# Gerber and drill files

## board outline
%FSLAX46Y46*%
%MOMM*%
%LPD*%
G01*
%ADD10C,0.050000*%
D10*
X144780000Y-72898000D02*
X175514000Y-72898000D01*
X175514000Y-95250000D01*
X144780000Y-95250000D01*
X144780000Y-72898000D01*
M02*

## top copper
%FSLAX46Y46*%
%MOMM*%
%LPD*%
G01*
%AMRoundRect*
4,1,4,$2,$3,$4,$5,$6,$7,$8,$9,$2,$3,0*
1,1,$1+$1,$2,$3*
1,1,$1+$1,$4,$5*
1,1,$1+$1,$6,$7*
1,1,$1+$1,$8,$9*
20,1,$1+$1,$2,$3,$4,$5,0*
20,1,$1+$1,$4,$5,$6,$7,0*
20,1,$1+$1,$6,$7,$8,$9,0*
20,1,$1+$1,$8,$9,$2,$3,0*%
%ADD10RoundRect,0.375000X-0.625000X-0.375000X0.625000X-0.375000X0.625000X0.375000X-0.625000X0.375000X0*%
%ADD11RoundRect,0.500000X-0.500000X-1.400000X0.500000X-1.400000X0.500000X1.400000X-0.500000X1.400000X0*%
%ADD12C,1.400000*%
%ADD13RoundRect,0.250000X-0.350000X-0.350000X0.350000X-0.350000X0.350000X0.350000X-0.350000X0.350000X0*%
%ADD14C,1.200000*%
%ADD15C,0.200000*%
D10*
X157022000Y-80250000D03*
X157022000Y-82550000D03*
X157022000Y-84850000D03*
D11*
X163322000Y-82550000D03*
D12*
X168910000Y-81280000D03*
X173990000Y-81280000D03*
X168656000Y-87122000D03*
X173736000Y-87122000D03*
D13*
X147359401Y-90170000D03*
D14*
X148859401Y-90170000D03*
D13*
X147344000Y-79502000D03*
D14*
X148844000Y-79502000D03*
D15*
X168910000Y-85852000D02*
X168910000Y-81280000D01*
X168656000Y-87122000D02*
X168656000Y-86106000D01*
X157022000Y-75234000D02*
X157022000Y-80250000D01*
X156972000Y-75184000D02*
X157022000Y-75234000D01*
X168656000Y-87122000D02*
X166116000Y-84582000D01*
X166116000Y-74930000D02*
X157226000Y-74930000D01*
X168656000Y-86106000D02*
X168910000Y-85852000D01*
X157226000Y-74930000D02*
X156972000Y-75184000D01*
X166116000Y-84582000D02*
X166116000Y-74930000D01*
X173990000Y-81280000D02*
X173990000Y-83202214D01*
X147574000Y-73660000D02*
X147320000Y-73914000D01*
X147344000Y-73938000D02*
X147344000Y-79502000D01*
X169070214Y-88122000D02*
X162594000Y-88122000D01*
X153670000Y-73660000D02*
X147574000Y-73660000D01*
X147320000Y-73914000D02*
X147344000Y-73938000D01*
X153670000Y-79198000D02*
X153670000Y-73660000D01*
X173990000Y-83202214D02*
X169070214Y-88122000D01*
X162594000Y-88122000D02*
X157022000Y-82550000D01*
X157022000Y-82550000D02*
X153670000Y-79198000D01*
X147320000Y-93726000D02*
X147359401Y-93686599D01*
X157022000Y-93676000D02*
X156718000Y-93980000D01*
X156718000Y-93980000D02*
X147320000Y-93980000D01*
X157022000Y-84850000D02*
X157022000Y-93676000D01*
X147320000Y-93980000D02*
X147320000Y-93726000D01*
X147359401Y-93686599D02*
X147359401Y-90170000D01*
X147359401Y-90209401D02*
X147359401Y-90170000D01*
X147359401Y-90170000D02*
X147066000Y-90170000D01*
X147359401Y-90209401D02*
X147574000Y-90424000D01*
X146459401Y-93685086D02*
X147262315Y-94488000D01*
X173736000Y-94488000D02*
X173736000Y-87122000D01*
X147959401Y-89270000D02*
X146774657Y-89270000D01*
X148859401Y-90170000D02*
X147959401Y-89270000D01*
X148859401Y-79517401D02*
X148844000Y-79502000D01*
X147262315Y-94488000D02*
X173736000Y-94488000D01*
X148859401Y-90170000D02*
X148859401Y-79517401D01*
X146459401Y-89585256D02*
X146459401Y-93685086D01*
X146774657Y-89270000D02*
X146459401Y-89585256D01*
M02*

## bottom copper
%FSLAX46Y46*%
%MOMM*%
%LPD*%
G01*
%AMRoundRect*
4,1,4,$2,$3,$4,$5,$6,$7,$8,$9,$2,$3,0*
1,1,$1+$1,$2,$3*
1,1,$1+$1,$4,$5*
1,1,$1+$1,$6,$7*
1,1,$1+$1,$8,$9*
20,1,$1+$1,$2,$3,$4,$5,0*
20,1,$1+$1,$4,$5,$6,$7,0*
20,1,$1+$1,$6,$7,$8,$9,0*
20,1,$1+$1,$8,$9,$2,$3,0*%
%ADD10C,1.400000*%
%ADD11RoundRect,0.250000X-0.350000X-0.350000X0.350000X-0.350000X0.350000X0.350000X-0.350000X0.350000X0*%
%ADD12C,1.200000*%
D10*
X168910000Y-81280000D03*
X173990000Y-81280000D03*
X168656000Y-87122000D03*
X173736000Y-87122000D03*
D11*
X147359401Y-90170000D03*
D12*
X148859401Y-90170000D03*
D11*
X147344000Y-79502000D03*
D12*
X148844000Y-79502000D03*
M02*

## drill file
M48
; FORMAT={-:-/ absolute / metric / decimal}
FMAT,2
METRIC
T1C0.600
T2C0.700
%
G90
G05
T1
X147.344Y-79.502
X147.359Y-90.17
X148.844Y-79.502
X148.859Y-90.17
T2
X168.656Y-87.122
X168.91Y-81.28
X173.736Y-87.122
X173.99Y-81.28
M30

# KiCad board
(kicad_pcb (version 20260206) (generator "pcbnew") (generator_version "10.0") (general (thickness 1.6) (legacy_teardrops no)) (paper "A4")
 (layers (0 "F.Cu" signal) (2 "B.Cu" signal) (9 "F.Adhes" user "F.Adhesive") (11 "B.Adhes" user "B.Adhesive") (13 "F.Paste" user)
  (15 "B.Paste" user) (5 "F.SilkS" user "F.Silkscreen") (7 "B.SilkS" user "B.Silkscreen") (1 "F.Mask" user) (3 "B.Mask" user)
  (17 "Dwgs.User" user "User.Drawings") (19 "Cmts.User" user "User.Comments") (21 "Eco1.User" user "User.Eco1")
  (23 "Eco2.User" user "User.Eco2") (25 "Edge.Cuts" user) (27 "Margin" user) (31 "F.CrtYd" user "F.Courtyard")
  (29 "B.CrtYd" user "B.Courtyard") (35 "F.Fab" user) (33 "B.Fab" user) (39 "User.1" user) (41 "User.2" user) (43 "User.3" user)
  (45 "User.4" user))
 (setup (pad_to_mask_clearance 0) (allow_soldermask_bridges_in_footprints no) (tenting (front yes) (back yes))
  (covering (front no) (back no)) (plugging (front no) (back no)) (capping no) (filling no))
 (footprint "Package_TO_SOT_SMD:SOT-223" (layer "F.Cu") (at 160.172 82.55)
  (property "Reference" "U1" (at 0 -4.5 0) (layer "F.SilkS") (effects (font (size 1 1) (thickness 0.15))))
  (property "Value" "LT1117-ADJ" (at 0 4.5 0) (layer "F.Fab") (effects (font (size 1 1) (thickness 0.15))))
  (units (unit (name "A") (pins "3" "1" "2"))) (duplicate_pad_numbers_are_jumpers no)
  (pad "1" smd roundrect (at -3.15 -2.3) (size 2 1.5) (layers "F.Cu" "F.Mask" "F.Paste") (roundrect_rratio 0.25) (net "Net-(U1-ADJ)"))
  (pad "2" smd roundrect (at -3.15 0) (size 2 1.5) (layers "F.Cu" "F.Mask" "F.Paste") (roundrect_rratio 0.25) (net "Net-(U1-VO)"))
  (pad "3" smd roundrect (at -3.15 2.3) (size 2 1.5) (layers "F.Cu" "F.Mask" "F.Paste") (roundrect_rratio 0.25) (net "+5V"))
  (pad "4" smd roundrect (at 3.15 0) (size 2 3.8) (layers "F.Cu" "F.Mask" "F.Paste") (roundrect_rratio 0.25)))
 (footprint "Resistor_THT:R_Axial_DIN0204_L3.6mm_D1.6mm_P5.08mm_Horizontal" (layer "F.Cu") (at 168.91 81.28)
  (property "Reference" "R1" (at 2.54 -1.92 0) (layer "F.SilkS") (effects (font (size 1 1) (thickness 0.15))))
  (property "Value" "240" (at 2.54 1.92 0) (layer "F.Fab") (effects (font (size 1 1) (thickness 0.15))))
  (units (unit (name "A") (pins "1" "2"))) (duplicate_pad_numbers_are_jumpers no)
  (pad "1" thru_hole circle (at 0 0) (size 1.4 1.4) (drill 0.7) (layers "*.Cu" "*.Mask") (remove_unused_layers no) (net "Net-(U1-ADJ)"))
  (pad "2" thru_hole circle (at 5.08 0) (size 1.4 1.4) (drill 0.7) (layers "*.Cu" "*.Mask") (remove_unused_layers no) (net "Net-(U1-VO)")))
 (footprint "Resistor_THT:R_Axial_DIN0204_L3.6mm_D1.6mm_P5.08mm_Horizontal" (layer "F.Cu") (at 168.656 87.122)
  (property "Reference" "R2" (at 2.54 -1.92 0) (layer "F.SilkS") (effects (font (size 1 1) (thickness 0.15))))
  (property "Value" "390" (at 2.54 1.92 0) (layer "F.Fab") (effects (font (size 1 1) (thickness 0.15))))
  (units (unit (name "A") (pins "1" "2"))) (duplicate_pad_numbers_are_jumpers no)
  (pad "1" thru_hole circle (at 0 0) (size 1.4 1.4) (drill 0.7) (layers "*.Cu" "*.Mask") (remove_unused_layers no) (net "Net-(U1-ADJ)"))
  (pad "2" thru_hole circle (at 5.08 0) (size 1.4 1.4) (drill 0.7) (layers "*.Cu" "*.Mask") (remove_unused_layers no) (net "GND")))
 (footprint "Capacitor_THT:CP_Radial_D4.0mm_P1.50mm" (layer "F.Cu") (at 147.359401 90.17)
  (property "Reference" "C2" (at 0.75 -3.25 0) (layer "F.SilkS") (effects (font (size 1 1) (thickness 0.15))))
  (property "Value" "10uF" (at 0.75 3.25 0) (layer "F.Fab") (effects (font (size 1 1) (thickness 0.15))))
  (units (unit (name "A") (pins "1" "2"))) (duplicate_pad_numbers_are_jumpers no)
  (pad "1" thru_hole roundrect (at 0 0) (size 1.2 1.2) (drill 0.6) (layers "*.Cu" "*.Mask") (remove_unused_layers no)
   (roundrect_rratio 0.208333) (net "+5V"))
  (pad "2" thru_hole circle (at 1.5 0) (size 1.2 1.2) (drill 0.6) (layers "*.Cu" "*.Mask") (remove_unused_layers no) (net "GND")))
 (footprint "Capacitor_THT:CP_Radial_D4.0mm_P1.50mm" (layer "F.Cu") (at 147.344 79.502)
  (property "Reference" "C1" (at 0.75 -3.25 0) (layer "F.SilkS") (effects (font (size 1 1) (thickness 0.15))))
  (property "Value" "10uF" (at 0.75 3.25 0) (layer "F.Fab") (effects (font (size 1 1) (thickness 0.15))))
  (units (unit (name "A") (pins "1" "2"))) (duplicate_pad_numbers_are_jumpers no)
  (pad "1" thru_hole roundrect (at 0 0) (size 1.2 1.2) (drill 0.6) (layers "*.Cu" "*.Mask") (remove_unused_layers no)
   (roundrect_rratio 0.208333) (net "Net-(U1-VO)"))
  (pad "2" thru_hole circle (at 1.5 0) (size 1.2 1.2) (drill 0.6) (layers "*.Cu" "*.Mask") (remove_unused_layers no) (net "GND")))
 (gr_rect (start 144.78 72.898) (end 175.514 95.25) (stroke (width 0.05) (type default)) (fill no) (layer "Edge.Cuts"))
 (segment (start 168.91 85.852) (end 168.91 81.28) (width 0.2) (layer "F.Cu") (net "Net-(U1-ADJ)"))
 (segment (start 168.656 87.122) (end 168.656 86.106) (width 0.2) (layer "F.Cu") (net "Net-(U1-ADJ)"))
 (segment (start 157.022 75.234) (end 157.022 80.25) (width 0.2) (layer "F.Cu") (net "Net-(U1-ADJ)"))
 (segment (start 156.972 75.184) (end 157.022 75.234) (width 0.2) (layer "F.Cu") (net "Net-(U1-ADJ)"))
 (segment (start 168.656 87.122) (end 166.116 84.582) (width 0.2) (layer "F.Cu") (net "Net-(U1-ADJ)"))
 (segment (start 166.116 74.93) (end 157.226 74.93) (width 0.2) (layer "F.Cu") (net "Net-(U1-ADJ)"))
 (segment (start 168.656 86.106) (end 168.91 85.852) (width 0.2) (layer "F.Cu") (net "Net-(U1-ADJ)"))
 (segment (start 157.226 74.93) (end 156.972 75.184) (width 0.2) (layer "F.Cu") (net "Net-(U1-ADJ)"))
 (segment (start 166.116 84.582) (end 166.116 74.93) (width 0.2) (layer "F.Cu") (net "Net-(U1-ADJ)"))
 (segment (start 173.99 81.28) (end 173.99 83.202214) (width 0.2) (layer "F.Cu") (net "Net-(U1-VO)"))
 (segment (start 147.574 73.66) (end 147.32 73.914) (width 0.2) (layer "F.Cu") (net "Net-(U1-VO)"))
 (segment (start 147.344 73.938) (end 147.344 79.502) (width 0.2) (layer "F.Cu") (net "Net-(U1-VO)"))
 (segment (start 169.070214 88.122) (end 162.594 88.122) (width 0.2) (layer "F.Cu") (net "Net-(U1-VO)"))
 (segment (start 153.67 73.66) (end 147.574 73.66) (width 0.2) (layer "F.Cu") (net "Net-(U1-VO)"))
 (segment (start 147.32 73.914) (end 147.344 73.938) (width 0.2) (layer "F.Cu") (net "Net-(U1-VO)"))
 (segment (start 153.67 79.198) (end 153.67 73.66) (width 0.2) (layer "F.Cu") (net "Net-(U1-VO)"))
 (segment (start 173.99 83.202214) (end 169.070214 88.122) (width 0.2) (layer "F.Cu") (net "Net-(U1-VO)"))
 (segment (start 162.594 88.122) (end 157.022 82.55) (width 0.2) (layer "F.Cu") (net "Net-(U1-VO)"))
 (segment (start 157.022 82.55) (end 153.67 79.198) (width 0.2) (layer "F.Cu") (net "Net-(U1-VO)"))
 (segment (start 147.32 93.726) (end 147.359401 93.686599) (width 0.2) (layer "F.Cu") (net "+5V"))
 (segment (start 157.022 93.676) (end 156.718 93.98) (width 0.2) (layer "F.Cu") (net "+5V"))
 (segment (start 156.718 93.98) (end 147.32 93.98) (width 0.2) (layer "F.Cu") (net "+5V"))
 (segment (start 157.022 84.85) (end 157.022 93.676) (width 0.2) (layer "F.Cu") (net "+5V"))
 (segment (start 147.32 93.98) (end 147.32 93.726) (width 0.2) (layer "F.Cu") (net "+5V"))
 (segment (start 147.359401 93.686599) (end 147.359401 90.17) (width 0.2) (layer "F.Cu") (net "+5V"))
 (segment (start 147.359401 90.209401) (end 147.359401 90.17) (width 0.2) (layer "F.Cu") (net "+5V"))
 (segment (start 147.359401 90.17) (end 147.066 90.17) (width 0.2) (layer "F.Cu") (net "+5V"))
 (segment (start 147.359401 90.209401) (end 147.574 90.424) (width 0.2) (layer "F.Cu") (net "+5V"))
 (segment (start 146.459401 93.685086) (end 147.262315 94.488) (width 0.2) (layer "F.Cu") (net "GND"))
 (segment (start 173.736 94.488) (end 173.736 87.122) (width 0.2) (layer "F.Cu") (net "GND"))
 (segment (start 147.959401 89.27) (end 146.774657 89.27) (width 0.2) (layer "F.Cu") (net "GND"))
 (segment (start 148.859401 90.17) (end 147.959401 89.27) (width 0.2) (layer "F.Cu") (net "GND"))
 (segment (start 148.859401 79.517401) (end 148.844 79.502) (width 0.2) (layer "F.Cu") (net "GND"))
 (segment (start 147.262315 94.488) (end 173.736 94.488) (width 0.2) (layer "F.Cu") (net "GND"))
 (segment (start 148.859401 90.17) (end 148.859401 79.517401) (width 0.2) (layer "F.Cu") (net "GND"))
 (segment (start 146.459401 89.585256) (end 146.459401 93.685086) (width 0.2) (layer "F.Cu") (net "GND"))
 (segment (start 146.774657 89.27) (end 146.459401 89.585256) (width 0.2) (layer "F.Cu") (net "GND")))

